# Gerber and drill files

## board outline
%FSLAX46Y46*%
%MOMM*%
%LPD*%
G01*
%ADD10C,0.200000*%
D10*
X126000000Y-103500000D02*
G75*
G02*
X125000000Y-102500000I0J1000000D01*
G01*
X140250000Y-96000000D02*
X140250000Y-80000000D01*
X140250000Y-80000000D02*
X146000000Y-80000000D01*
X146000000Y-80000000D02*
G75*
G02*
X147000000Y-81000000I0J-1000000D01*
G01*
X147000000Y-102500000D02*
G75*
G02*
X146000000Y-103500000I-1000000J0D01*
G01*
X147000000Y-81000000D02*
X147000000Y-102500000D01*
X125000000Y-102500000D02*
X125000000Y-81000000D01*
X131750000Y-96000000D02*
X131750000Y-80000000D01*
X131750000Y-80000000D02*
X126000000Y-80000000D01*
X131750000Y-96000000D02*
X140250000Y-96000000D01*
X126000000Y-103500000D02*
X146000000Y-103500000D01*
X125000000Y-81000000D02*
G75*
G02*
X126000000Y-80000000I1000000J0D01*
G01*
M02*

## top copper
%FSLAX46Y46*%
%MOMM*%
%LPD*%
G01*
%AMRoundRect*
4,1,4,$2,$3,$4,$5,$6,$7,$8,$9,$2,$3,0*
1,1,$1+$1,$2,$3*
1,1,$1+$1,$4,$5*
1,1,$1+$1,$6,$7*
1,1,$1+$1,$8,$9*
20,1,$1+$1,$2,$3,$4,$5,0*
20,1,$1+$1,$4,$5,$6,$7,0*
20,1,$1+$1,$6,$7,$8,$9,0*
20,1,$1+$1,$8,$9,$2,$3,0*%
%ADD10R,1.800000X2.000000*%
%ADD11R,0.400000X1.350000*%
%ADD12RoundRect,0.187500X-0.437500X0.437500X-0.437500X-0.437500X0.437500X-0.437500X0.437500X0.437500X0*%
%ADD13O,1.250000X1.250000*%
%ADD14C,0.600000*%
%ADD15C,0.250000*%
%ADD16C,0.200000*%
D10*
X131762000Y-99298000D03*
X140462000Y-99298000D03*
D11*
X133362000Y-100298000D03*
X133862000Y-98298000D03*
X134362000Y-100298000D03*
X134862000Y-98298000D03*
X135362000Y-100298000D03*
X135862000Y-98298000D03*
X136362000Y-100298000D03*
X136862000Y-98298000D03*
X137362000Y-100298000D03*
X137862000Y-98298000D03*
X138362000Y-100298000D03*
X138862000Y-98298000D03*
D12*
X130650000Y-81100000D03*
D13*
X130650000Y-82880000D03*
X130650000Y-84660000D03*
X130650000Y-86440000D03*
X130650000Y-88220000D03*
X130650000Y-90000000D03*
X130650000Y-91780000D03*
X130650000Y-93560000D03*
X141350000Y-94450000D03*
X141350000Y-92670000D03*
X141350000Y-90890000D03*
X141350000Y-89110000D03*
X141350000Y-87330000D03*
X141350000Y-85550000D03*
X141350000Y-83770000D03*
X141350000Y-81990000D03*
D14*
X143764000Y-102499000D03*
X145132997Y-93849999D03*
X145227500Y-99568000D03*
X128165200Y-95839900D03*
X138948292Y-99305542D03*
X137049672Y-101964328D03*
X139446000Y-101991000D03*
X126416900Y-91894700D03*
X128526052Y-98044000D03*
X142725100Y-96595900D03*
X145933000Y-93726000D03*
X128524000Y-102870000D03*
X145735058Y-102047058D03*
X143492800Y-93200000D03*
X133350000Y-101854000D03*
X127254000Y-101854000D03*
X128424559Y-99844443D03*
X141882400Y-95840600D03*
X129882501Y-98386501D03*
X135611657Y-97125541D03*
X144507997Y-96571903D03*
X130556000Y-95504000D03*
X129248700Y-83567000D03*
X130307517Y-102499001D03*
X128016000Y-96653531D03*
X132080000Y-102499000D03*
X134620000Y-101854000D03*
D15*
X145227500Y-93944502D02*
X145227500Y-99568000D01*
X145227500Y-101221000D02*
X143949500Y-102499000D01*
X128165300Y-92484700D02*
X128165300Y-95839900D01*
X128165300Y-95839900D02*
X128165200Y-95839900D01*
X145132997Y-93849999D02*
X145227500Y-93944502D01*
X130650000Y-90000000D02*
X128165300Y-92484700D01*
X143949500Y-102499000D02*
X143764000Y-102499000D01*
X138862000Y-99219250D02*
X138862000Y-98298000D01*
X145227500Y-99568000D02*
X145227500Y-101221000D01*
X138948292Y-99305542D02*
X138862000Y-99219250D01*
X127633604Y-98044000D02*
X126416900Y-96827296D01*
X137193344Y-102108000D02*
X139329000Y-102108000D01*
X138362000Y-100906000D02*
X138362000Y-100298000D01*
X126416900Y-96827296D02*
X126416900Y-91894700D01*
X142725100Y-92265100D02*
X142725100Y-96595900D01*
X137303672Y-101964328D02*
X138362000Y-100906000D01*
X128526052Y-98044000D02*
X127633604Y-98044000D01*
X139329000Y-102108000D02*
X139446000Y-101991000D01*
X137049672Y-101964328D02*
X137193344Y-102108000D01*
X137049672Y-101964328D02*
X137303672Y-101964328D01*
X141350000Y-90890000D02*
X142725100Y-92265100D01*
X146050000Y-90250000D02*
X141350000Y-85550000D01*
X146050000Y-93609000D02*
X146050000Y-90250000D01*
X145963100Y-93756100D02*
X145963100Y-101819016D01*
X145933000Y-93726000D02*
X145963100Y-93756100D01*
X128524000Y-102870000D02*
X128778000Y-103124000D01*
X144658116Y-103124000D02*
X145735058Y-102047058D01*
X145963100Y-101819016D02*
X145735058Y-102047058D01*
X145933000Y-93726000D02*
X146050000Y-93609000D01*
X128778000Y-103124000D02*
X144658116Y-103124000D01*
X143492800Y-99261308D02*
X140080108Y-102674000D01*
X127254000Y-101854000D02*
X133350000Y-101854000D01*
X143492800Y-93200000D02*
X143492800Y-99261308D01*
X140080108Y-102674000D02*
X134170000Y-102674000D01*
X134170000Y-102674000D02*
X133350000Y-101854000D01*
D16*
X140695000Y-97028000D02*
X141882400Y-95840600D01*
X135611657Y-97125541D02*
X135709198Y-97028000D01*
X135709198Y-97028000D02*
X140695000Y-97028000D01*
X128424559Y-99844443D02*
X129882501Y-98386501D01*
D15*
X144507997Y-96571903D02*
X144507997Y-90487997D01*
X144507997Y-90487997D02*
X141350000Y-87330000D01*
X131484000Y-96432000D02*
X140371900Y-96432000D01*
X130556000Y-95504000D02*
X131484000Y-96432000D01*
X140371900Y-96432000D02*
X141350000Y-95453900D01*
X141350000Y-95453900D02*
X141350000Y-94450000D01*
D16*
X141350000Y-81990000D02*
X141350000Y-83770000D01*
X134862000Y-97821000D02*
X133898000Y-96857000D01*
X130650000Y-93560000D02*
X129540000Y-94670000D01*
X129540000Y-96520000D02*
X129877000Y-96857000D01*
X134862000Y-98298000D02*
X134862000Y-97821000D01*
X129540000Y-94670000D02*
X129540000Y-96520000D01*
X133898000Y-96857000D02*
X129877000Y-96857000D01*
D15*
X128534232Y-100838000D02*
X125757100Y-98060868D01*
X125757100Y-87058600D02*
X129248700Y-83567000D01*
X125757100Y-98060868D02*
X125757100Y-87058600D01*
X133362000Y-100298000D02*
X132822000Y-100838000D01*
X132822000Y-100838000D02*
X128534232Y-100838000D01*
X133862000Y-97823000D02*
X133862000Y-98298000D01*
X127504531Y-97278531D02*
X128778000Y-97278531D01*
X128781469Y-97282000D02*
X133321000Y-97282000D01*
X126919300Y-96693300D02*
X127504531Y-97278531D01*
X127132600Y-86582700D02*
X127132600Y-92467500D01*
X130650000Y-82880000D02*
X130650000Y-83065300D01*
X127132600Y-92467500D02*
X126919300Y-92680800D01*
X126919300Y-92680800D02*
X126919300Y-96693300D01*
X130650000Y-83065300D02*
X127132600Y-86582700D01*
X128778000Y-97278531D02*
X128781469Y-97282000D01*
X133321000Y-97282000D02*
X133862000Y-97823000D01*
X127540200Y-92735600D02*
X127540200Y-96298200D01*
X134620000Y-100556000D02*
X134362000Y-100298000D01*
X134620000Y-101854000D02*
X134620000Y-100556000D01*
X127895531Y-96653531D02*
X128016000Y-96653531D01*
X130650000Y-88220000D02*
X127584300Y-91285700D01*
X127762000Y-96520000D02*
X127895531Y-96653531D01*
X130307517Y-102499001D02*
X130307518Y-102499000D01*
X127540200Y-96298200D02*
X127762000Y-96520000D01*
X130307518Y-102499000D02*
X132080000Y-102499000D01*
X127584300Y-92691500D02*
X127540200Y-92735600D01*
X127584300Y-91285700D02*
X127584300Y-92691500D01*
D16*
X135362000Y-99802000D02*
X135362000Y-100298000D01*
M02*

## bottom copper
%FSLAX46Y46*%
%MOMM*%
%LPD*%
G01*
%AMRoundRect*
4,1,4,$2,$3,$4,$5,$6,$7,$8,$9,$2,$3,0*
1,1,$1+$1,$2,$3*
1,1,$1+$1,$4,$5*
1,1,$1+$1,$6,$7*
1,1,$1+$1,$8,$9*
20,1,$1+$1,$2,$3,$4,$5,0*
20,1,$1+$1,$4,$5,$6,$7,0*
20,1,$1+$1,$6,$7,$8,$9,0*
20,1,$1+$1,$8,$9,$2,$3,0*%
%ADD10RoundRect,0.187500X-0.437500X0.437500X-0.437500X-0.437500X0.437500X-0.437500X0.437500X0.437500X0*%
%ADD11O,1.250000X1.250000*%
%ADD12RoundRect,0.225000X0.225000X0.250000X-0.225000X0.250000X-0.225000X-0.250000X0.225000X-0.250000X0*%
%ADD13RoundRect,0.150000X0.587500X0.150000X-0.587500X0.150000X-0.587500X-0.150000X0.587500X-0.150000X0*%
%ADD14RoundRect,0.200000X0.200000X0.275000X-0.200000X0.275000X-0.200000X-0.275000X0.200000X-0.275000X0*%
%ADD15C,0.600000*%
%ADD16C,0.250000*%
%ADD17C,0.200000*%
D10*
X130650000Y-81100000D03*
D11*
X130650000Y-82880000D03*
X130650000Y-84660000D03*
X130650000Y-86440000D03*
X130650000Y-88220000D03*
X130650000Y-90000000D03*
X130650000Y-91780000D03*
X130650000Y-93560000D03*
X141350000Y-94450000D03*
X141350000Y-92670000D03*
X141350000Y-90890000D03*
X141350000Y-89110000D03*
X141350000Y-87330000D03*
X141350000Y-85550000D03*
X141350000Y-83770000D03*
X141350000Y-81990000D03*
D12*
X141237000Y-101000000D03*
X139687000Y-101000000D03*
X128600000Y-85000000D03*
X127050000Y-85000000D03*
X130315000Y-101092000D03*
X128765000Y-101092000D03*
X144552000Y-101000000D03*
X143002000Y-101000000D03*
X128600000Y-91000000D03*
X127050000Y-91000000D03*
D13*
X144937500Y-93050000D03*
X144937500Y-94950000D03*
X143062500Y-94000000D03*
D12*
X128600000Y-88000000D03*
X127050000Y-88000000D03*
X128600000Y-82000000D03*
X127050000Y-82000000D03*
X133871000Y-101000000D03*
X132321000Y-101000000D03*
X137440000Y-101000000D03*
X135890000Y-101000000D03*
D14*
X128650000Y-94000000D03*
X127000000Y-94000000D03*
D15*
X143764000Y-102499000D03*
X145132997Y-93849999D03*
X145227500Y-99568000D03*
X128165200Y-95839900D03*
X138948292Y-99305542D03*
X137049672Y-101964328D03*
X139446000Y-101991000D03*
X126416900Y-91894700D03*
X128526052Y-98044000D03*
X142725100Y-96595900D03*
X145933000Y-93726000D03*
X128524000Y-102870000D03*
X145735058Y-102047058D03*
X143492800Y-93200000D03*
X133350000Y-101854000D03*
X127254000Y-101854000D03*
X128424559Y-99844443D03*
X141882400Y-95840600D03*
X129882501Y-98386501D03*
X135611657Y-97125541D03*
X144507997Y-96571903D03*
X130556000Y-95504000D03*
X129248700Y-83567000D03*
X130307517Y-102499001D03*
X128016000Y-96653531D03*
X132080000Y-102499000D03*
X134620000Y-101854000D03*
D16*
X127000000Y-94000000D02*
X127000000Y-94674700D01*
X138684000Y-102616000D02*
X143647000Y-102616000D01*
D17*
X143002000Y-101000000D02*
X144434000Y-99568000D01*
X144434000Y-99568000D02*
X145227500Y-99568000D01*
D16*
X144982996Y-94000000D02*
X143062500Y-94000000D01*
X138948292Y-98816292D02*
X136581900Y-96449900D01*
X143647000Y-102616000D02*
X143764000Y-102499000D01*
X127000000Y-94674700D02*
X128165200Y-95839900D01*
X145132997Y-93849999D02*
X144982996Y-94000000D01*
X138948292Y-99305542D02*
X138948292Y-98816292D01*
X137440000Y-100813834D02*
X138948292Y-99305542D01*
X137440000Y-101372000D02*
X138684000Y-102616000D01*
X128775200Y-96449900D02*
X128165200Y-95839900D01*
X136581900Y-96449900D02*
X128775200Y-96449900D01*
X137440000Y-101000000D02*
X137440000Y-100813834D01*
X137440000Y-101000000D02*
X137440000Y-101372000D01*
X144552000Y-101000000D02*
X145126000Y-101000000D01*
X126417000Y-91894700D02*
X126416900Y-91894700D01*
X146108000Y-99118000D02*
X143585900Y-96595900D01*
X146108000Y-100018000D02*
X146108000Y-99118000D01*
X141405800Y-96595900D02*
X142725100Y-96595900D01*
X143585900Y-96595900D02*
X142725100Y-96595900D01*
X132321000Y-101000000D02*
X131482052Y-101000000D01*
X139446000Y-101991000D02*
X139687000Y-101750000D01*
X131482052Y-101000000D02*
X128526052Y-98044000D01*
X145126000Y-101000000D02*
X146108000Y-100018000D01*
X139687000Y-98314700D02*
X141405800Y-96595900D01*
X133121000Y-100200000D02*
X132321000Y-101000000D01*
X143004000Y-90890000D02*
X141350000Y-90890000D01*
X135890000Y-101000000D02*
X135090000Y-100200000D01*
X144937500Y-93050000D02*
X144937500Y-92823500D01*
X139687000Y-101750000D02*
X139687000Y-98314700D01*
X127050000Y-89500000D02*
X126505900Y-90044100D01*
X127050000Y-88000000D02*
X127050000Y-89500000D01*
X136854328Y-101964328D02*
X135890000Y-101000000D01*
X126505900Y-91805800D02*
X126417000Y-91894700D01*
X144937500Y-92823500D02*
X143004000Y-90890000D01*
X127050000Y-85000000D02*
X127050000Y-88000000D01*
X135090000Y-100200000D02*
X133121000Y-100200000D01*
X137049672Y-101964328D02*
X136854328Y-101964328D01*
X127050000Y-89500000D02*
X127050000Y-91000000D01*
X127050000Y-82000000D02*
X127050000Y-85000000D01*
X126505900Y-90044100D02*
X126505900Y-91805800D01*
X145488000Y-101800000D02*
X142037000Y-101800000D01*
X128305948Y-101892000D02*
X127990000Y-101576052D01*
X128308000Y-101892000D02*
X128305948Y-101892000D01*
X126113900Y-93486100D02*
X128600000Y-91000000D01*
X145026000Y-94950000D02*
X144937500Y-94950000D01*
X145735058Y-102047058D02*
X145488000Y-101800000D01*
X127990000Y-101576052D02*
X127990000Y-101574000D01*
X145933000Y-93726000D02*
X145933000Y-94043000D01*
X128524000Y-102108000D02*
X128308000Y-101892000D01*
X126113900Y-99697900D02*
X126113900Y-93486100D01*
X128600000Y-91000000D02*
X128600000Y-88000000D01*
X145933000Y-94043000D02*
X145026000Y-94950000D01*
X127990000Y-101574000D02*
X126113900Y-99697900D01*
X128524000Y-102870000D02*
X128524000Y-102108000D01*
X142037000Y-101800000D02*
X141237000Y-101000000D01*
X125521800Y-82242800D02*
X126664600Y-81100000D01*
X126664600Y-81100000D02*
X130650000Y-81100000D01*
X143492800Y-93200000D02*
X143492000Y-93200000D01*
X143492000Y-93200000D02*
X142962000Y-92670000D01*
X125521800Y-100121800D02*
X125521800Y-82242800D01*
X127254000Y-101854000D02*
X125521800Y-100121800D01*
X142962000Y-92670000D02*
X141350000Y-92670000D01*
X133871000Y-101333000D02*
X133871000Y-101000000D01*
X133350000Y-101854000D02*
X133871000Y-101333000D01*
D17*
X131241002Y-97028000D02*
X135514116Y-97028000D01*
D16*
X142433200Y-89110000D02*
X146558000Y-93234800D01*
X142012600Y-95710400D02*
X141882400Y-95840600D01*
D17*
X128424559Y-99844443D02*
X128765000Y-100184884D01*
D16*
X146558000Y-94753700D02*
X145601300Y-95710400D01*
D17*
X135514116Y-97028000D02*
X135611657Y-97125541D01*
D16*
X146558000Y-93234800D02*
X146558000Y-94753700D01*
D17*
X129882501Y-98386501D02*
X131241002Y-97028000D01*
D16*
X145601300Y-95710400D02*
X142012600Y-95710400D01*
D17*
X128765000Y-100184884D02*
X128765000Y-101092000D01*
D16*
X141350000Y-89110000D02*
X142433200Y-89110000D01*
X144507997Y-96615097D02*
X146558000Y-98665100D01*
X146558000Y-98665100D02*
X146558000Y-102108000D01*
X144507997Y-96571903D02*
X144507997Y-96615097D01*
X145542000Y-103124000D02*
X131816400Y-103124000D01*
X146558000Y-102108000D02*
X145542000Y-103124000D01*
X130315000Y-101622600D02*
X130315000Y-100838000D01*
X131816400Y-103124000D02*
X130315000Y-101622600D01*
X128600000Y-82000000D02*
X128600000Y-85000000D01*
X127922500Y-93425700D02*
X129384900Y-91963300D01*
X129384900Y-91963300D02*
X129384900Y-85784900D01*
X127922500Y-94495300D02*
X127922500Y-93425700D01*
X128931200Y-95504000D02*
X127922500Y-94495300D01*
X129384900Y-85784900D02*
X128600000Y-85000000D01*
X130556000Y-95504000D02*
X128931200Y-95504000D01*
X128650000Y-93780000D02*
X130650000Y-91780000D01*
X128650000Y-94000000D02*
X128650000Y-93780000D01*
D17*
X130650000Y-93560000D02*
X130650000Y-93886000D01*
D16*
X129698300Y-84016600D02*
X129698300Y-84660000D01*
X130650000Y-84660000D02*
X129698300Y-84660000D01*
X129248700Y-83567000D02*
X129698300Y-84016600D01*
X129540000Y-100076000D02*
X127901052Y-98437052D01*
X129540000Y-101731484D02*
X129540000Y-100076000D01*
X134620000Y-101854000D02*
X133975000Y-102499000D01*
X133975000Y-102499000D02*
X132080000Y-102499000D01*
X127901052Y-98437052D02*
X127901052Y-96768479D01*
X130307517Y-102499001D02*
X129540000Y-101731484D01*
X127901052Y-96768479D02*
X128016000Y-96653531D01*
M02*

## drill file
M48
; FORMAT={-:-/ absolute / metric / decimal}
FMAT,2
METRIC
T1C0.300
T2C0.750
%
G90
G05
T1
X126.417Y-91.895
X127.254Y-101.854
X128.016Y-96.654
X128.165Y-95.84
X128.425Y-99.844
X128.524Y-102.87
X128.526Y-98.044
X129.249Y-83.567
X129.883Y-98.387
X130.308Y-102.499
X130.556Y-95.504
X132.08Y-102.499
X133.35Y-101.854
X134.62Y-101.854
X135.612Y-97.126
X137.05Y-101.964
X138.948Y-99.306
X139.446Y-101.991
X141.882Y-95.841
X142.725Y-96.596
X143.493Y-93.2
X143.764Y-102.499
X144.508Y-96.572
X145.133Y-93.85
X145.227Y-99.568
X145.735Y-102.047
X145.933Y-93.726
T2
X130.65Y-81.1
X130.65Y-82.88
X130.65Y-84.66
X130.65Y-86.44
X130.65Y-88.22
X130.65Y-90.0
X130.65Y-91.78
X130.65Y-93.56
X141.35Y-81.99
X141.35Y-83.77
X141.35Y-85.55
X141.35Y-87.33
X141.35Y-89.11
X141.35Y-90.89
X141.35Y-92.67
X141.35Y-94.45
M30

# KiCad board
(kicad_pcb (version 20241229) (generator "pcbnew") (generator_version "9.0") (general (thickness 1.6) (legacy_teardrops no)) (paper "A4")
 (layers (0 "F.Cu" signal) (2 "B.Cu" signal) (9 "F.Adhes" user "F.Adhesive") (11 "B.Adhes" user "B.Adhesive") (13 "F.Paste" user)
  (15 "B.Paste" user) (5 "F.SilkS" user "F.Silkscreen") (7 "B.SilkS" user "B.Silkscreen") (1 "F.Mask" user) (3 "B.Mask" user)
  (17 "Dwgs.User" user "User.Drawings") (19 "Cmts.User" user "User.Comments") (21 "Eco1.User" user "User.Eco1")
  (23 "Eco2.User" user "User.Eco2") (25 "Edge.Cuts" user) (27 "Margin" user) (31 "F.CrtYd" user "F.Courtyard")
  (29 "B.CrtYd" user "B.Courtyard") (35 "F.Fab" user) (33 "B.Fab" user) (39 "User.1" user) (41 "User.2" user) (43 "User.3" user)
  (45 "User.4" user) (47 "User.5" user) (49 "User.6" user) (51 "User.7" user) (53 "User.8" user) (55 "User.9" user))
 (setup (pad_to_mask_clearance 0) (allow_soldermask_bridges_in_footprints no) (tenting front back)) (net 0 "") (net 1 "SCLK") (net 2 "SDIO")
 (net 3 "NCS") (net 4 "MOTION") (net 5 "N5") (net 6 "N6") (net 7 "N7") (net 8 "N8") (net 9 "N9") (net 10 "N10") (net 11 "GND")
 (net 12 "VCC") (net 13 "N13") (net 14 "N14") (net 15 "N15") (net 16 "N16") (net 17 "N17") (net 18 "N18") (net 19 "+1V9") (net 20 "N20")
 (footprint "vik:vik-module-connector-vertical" (layer "F.Cu") (at 136.112 99.298)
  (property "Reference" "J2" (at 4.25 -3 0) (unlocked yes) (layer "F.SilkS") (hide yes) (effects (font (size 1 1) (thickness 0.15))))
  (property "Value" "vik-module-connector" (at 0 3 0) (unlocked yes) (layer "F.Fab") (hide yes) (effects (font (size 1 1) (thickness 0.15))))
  (pad "" smd rect (at -4.35 0) (size 1.8 2) (layers "F.Cu" "F.Mask" "F.Paste") (thermal_bridge_angle 45))
  (pad "" smd rect (at 4.35 0) (size 1.8 2) (layers "F.Cu" "F.Mask" "F.Paste") (thermal_bridge_angle 45))
  (pad "1" smd rect (at -2.75 1) (size 0.4 1.35) (layers "F.Cu" "F.Mask" "F.Paste") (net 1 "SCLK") (thermal_bridge_angle 45))
  (pad "2" smd rect (at -2.25 -1) (size 0.4 1.35) (layers "F.Cu" "F.Mask" "F.Paste") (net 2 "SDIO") (thermal_bridge_angle 45))
  (pad "3" smd rect (at -1.75 1) (size 0.4 1.35) (layers "F.Cu" "F.Mask" "F.Paste") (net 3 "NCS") (thermal_bridge_angle 45))
  (pad "4" smd rect (at -1.25 -1) (size 0.4 1.35) (layers "F.Cu" "F.Mask" "F.Paste") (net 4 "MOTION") (thermal_bridge_angle 45))
  (pad "5" smd rect (at -0.75 1) (size 0.4 1.35) (layers "F.Cu" "F.Mask" "F.Paste") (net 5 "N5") (thermal_bridge_angle 45))
  (pad "6" smd rect (at -0.25 -1) (size 0.4 1.35) (layers "F.Cu" "F.Mask" "F.Paste") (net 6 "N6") (thermal_bridge_angle 45))
  (pad "7" smd rect (at 0.25 1) (size 0.4 1.35) (layers "F.Cu" "F.Mask" "F.Paste") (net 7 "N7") (thermal_bridge_angle 45))
  (pad "8" smd rect (at 0.75 -1) (size 0.4 1.35) (layers "F.Cu" "F.Mask" "F.Paste") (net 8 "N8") (thermal_bridge_angle 45))
  (pad "9" smd rect (at 1.25 1) (size 0.4 1.35) (layers "F.Cu" "F.Mask" "F.Paste") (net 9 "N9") (thermal_bridge_angle 45))
  (pad "10" smd rect (at 1.75 -1) (size 0.4 1.35) (layers "F.Cu" "F.Mask" "F.Paste") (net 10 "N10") (thermal_bridge_angle 45))
  (pad "11" smd rect (at 2.25 1) (size 0.4 1.35) (layers "F.Cu" "F.Mask" "F.Paste") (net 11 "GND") (thermal_bridge_angle 45))
  (pad "12" smd rect (at 2.75 -1) (size 0.4 1.35) (layers "F.Cu" "F.Mask" "F.Paste") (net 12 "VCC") (thermal_bridge_angle 45)))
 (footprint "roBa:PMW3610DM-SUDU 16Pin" (layer "F.Cu") (at 136 87.268 90)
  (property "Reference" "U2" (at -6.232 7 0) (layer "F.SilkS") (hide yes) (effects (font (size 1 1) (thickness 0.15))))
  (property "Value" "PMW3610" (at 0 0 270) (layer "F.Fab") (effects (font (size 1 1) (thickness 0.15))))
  (pad "1" thru_hole roundrect (at 6.168 -5.35 270) (size 1.25 1.25) (drill 0.75) (layers "*.Cu" "*.Mask") (remove_unused_layers no)
   (roundrect_rratio 0.15) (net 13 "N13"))
  (pad "2" thru_hole oval (at 4.388 -5.35 270) (size 1.25 1.25) (drill 0.75) (layers "*.Cu" "*.Mask") (remove_unused_layers no)
   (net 2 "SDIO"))
  (pad "3" thru_hole oval (at 2.608 -5.35 270) (size 1.25 1.25) (drill 0.75) (layers "*.Cu" "*.Mask") (remove_unused_layers no)
   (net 1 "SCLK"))
  (pad "4" thru_hole oval (at 0.828 -5.35 270) (size 1.25 1.25) (drill 0.75) (layers "*.Cu" "*.Mask") (remove_unused_layers no)
   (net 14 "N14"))
  (pad "5" thru_hole oval (at -0.952 -5.35 270) (size 1.25 1.25) (drill 0.75) (layers "*.Cu" "*.Mask") (remove_unused_layers no)
   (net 3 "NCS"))
  (pad "6" thru_hole oval (at -2.732 -5.35 270) (size 1.25 1.25) (drill 0.75) (layers "*.Cu" "*.Mask") (remove_unused_layers no)
   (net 12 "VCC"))
  (pad "7" thru_hole oval (at -4.512 -5.35 270) (size 1.25 1.25) (drill 0.75) (layers "*.Cu" "*.Mask") (remove_unused_layers no)
   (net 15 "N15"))
  (pad "8" thru_hole oval (at -6.292 -5.35 270) (size 1.25 1.25) (drill 0.75) (layers "*.Cu" "*.Mask") (remove_unused_layers no)
   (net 4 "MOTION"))
  (pad "9" thru_hole oval (at -7.182 5.35 270) (size 1.25 1.25) (drill 0.75) (layers "*.Cu" "*.Mask") (remove_unused_layers no)
   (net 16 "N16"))
  (pad "10" thru_hole oval (at -5.402 5.35 270) (size 1.25 1.25) (drill 0.75) (layers "*.Cu" "*.Mask") (remove_unused_layers no)
   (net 13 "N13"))
  (pad "11" thru_hole oval (at -3.622 5.35 270) (size 1.25 1.25) (drill 0.75) (layers "*.Cu" "*.Mask") (remove_unused_layers no)
   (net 11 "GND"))
  (pad "12" thru_hole oval (at -1.842 5.35 270) (size 1.25 1.25) (drill 0.75) (layers "*.Cu" "*.Mask") (remove_unused_layers no)
   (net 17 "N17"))
  (pad "13" thru_hole oval (at -0.062 5.35 270) (size 1.25 1.25) (drill 0.75) (layers "*.Cu" "*.Mask") (remove_unused_layers no)
   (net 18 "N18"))
  (pad "14" thru_hole oval (at 1.718 5.35 270) (size 1.25 1.25) (drill 0.75) (layers "*.Cu" "*.Mask") (remove_unused_layers no)
   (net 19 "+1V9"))
  (pad "15" thru_hole oval (at 3.498 5.35 270) (size 1.25 1.25) (drill 0.75) (layers "*.Cu" "*.Mask") (remove_unused_layers no)
   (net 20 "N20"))
  (pad "16" thru_hole oval (at 5.278 5.35 270) (size 1.25 1.25) (drill 0.75) (layers "*.Cu" "*.Mask") (remove_unused_layers no)
   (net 20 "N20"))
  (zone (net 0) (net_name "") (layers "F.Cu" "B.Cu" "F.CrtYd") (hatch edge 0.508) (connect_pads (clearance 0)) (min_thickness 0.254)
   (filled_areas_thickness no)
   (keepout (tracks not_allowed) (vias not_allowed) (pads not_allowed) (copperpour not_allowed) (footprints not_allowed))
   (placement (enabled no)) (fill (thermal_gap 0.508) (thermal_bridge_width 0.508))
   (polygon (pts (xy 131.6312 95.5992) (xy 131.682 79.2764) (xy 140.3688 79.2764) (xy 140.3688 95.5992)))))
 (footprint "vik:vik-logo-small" (layer "F.Cu") (at 143.5 84.5)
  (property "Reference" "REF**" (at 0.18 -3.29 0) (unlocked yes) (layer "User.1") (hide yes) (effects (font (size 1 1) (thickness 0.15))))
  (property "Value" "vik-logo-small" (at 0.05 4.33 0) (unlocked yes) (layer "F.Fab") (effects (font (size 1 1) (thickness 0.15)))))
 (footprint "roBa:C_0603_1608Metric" (layer "B.Cu") (at 140.462 101 180)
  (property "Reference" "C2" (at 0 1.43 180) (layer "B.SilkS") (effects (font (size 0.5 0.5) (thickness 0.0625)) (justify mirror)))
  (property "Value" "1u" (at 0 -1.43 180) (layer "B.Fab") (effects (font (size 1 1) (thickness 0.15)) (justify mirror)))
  (pad "1" smd roundrect (at -0.775 0 180) (size 0.9 0.95) (layers "B.Cu" "B.Mask" "B.Paste") (roundrect_rratio 0.25) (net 19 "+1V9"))
  (pad "2" smd roundrect (at 0.775 0 180) (size 0.9 0.95) (layers "B.Cu" "B.Mask" "B.Paste") (roundrect_rratio 0.25) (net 11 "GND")))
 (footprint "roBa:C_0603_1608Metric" (layer "B.Cu") (at 127.825 85 180)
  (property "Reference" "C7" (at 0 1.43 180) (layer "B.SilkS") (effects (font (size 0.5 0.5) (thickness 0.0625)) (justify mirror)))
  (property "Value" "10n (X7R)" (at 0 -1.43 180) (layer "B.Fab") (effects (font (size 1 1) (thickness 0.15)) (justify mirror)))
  (pad "1" smd roundrect (at -0.775 0 180) (size 0.9 0.95) (layers "B.Cu" "B.Mask" "B.Paste") (roundrect_rratio 0.25) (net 16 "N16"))
  (pad "2" smd roundrect (at 0.775 0 180) (size 0.9 0.95) (layers "B.Cu" "B.Mask" "B.Paste") (roundrect_rratio 0.25) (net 11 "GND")))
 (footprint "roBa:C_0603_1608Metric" (layer "B.Cu") (at 129.54 101.092 180)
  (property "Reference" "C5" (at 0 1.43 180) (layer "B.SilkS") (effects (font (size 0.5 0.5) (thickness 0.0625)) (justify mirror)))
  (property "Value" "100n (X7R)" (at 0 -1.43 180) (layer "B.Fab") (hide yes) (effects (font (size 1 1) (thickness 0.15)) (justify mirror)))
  (pad "1" smd roundrect (at -0.775 0 180) (size 0.9 0.95) (layers "B.Cu" "B.Mask" "B.Paste") (roundrect_rratio 0.25) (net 18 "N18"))
  (pad "2" smd roundrect (at 0.775 0 180) (size 0.9 0.95) (layers "B.Cu" "B.Mask" "B.Paste") (roundrect_rratio 0.25) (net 17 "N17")))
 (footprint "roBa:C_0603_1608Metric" (layer "B.Cu") (at 143.777 101 180)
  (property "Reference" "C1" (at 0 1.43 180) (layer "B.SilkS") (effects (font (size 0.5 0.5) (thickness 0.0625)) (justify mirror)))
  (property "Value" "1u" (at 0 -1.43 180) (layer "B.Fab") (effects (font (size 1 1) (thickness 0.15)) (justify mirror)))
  (pad "1" smd roundrect (at -0.775 0 180) (size 0.9 0.95) (layers "B.Cu" "B.Mask" "B.Paste") (roundrect_rratio 0.25) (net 11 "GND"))
  (pad "2" smd roundrect (at 0.775 0 180) (size 0.9 0.95) (layers "B.Cu" "B.Mask" "B.Paste") (roundrect_rratio 0.25) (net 12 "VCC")))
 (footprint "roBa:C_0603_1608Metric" (layer "B.Cu") (at 127.825 91 180)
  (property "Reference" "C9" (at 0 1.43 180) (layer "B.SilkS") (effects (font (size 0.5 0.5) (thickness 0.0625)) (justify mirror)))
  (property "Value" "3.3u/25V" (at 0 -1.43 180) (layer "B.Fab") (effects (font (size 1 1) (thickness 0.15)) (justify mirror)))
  (pad "1" smd roundrect (at -0.775 0 180) (size 0.9 0.95) (layers "B.Cu" "B.Mask" "B.Paste") (roundrect_rratio 0.25) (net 19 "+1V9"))
  (pad "2" smd roundrect (at 0.775 0 180) (size 0.9 0.95) (layers "B.Cu" "B.Mask" "B.Paste") (roundrect_rratio 0.25) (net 11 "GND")))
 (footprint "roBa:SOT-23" (layer "B.Cu") (at 144 94 180)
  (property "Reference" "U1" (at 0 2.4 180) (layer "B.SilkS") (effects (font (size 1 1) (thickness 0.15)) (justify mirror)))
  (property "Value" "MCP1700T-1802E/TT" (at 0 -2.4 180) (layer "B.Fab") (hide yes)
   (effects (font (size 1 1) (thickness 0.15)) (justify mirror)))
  (pad "1" smd roundrect (at -0.9375 0.95 180) (size 1.475 0.6) (layers "B.Cu" "B.Mask" "B.Paste") (roundrect_rratio 0.25) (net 11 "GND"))
  (pad "2" smd roundrect (at -0.9375 -0.95 180) (size 1.475 0.6) (layers "B.Cu" "B.Mask" "B.Paste") (roundrect_rratio 0.25) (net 19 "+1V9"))
  (pad "3" smd roundrect (at 0.9375 0 180) (size 1.475 0.6) (layers "B.Cu" "B.Mask" "B.Paste") (roundrect_rratio 0.25) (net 12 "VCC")))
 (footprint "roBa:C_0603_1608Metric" (layer "B.Cu") (at 127.825 88 180)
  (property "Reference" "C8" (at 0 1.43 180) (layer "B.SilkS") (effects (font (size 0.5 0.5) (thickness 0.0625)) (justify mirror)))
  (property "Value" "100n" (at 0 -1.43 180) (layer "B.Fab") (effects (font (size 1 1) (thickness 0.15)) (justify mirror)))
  (pad "1" smd roundrect (at -0.775 0 180) (size 0.9 0.95) (layers "B.Cu" "B.Mask" "B.Paste") (roundrect_rratio 0.25) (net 19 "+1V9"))
  (pad "2" smd roundrect (at 0.775 0 180) (size 0.9 0.95) (layers "B.Cu" "B.Mask" "B.Paste") (roundrect_rratio 0.25) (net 11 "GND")))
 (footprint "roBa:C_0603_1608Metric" (layer "B.Cu") (at 127.825 82 180)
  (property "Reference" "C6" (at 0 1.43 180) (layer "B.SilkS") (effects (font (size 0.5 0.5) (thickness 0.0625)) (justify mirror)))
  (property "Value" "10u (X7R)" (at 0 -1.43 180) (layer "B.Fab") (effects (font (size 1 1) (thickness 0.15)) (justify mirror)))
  (pad "1" smd roundrect (at -0.775 0 180) (size 0.9 0.95) (layers "B.Cu" "B.Mask" "B.Paste") (roundrect_rratio 0.25) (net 16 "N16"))
  (pad "2" smd roundrect (at 0.775 0 180) (size 0.9 0.95) (layers "B.Cu" "B.Mask" "B.Paste") (roundrect_rratio 0.25) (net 11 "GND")))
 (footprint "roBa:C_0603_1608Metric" (layer "B.Cu") (at 133.096 101 180)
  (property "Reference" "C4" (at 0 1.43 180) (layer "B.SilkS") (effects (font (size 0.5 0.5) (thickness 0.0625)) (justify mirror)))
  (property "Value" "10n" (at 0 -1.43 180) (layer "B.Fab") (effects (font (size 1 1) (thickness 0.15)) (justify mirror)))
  (pad "1" smd roundrect (at -0.775 0 180) (size 0.9 0.95) (layers "B.Cu" "B.Mask" "B.Paste") (roundrect_rratio 0.25) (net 13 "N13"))
  (pad "2" smd roundrect (at 0.775 0 180) (size 0.9 0.95) (layers "B.Cu" "B.Mask" "B.Paste") (roundrect_rratio 0.25) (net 11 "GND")))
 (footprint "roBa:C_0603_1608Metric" (layer "B.Cu") (at 136.665 101 180)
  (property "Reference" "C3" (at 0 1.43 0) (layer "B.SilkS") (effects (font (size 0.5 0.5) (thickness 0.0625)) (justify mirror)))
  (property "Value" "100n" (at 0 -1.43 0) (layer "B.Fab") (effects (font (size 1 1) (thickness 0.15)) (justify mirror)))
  (pad "1" smd roundrect (at -0.775 0 180) (size 0.9 0.95) (layers "B.Cu" "B.Mask" "B.Paste") (roundrect_rratio 0.25) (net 12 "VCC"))
  (pad "2" smd roundrect (at 0.775 0 180) (size 0.9 0.95) (layers "B.Cu" "B.Mask" "B.Paste") (roundrect_rratio 0.25) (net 11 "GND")))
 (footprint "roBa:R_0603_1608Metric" (layer "B.Cu") (at 127.825 94 180)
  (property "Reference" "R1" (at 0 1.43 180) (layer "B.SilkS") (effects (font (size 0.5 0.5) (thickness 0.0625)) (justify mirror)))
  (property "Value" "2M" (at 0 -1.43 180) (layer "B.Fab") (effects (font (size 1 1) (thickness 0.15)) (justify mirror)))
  (pad "1" smd roundrect (at -0.825 0 180) (size 0.8 0.95) (layers "B.Cu" "B.Mask" "B.Paste") (roundrect_rratio 0.25) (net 15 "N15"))
  (pad "2" smd roundrect (at 0.825 0 180) (size 0.8 0.95) (layers "B.Cu" "B.Mask" "B.Paste") (roundrect_rratio 0.25) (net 12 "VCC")))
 (gr_arc (start 126 103.5) (mid 125.292893 103.207107) (end 125 102.5) (stroke (width 0.2) (type default)) (layer "Edge.Cuts"))
 (gr_line (start 140.25 96) (end 140.25 80) (stroke (width 0.2) (type default)) (layer "Edge.Cuts"))
 (gr_line (start 140.25 80) (end 146 80) (stroke (width 0.2) (type default)) (layer "Edge.Cuts"))
 (gr_arc (start 146 80) (mid 146.707107 80.292893) (end 147 81) (stroke (width 0.2) (type default)) (layer "Edge.Cuts"))
 (gr_arc (start 147 102.5) (mid 146.707107 103.207107) (end 146 103.5) (stroke (width 0.2) (type default)) (layer "Edge.Cuts"))
 (gr_line (start 147 81) (end 147 102.5) (stroke (width 0.2) (type default)) (layer "Edge.Cuts"))
 (gr_line (start 125 102.5) (end 125 81) (stroke (width 0.2) (type default)) (layer "Edge.Cuts"))
 (gr_line (start 131.75 96) (end 131.75 80) (stroke (width 0.2) (type default)) (layer "Edge.Cuts"))
 (gr_line (start 131.75 80) (end 126 80) (stroke (width 0.2) (type default)) (layer "Edge.Cuts"))
 (gr_line (start 131.75 96) (end 140.25 96) (stroke (width 0.2) (type default)) (layer "Edge.Cuts"))
 (gr_line (start 126 103.5) (end 146 103.5) (stroke (width 0.2) (type default)) (layer "Edge.Cuts"))
 (gr_arc (start 125 81) (mid 125.292893 80.292893) (end 126 80) (stroke (width 0.2) (type default)) (layer "Edge.Cuts"))
 (segment (start 145.2275 93.944502) (end 145.2275 99.568) (width 0.25) (layer "F.Cu") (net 12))
 (segment (start 145.2275 101.221) (end 143.9495 102.499) (width 0.25) (layer "F.Cu") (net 12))
 (segment (start 128.1653 92.4847) (end 128.1653 95.8399) (width 0.25) (layer "F.Cu") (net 12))
 (segment (start 128.1653 95.8399) (end 128.1652 95.8399) (width 0.25) (layer "F.Cu") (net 12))
 (segment (start 145.132997 93.849999) (end 145.2275 93.944502) (width 0.25) (layer "F.Cu") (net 12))
 (segment (start 130.65 90) (end 128.1653 92.4847) (width 0.25) (layer "F.Cu") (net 12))
 (segment (start 143.9495 102.499) (end 143.764 102.499) (width 0.25) (layer "F.Cu") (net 12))
 (segment (start 138.862 99.21925) (end 138.862 98.298) (width 0.25) (layer "F.Cu") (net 12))
 (segment (start 145.2275 99.568) (end 145.2275 101.221) (width 0.25) (layer "F.Cu") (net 12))
 (segment (start 138.948292 99.305542) (end 138.862 99.21925) (width 0.25) (layer "F.Cu") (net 12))
 (via (at 143.764 102.499) (size 0.6) (drill 0.3) (layers "F.Cu" "B.Cu") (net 12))
 (via (at 145.132997 93.849999) (size 0.6) (drill 0.3) (layers "F.Cu" "B.Cu") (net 12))
 (via (at 145.2275 99.568) (size 0.6) (drill 0.3) (layers "F.Cu" "B.Cu") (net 12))
 (via (at 128.1652 95.8399) (size 0.6) (drill 0.3) (layers "F.Cu" "B.Cu") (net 12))
 (via (at 138.948292 99.305542) (size 0.6) (drill 0.3) (layers "F.Cu" "B.Cu") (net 12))
 (segment (start 127 94) (end 127 94.6747) (width 0.25) (layer "B.Cu") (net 12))
 (segment (start 138.684 102.616) (end 143.647 102.616) (width 0.25) (layer "B.Cu") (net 12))
 (segment (start 143.002 101) (end 144.434 99.568) (width 0.2) (layer "B.Cu") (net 12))
 (segment (start 144.434 99.568) (end 145.2275 99.568) (width 0.2) (layer "B.Cu") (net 12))
 (segment (start 144.982996 94) (end 143.0625 94) (width 0.25) (layer "B.Cu") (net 12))
 (segment (start 138.948292 98.816292) (end 136.5819 96.4499) (width 0.25) (layer "B.Cu") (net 12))
 (segment (start 143.647 102.616) (end 143.764 102.499) (width 0.25) (layer "B.Cu") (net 12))
 (segment (start 127 94.6747) (end 128.1652 95.8399) (width 0.25) (layer "B.Cu") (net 12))
 (segment (start 145.132997 93.849999) (end 144.982996 94) (width 0.25) (layer "B.Cu") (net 12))
 (segment (start 138.948292 99.305542) (end 138.948292 98.816292) (width 0.25) (layer "B.Cu") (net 12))
 (segment (start 137.44 100.813834) (end 138.948292 99.305542) (width 0.25) (layer "B.Cu") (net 12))
 (segment (start 137.44 101.372) (end 138.684 102.616) (width 0.25) (layer "B.Cu") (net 12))
 (segment (start 128.7752 96.4499) (end 128.1652 95.8399) (width 0.25) (layer "B.Cu") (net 12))
 (segment (start 136.5819 96.4499) (end 128.7752 96.4499) (width 0.25) (layer "B.Cu") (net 12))
 (segment (start 137.44 101) (end 137.44 100.813834) (width 0.25) (layer "B.Cu") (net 12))
 (segment (start 137.44 101) (end 137.44 101.372) (width 0.25) (layer "B.Cu") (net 12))
 (segment (start 127.633604 98.044) (end 126.4169 96.827296) (width 0.25) (layer "F.Cu") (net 11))
 (segment (start 137.193344 102.108) (end 139.329 102.108) (width 0.25) (layer "F.Cu") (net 11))
 (segment (start 138.362 100.906) (end 138.362 100.298) (width 0.25) (layer "F.Cu") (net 11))
 (segment (start 126.4169 96.827296) (end 126.4169 91.8947) (width 0.25) (layer "F.Cu") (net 11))
 (segment (start 142.7251 92.2651) (end 142.7251 96.5959) (width 0.25) (layer "F.Cu") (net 11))
 (segment (start 137.303672 101.964328) (end 138.362 100.906) (width 0.25) (layer "F.Cu") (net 11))
 (segment (start 128.526052 98.044) (end 127.633604 98.044) (width 0.25) (layer "F.Cu") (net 11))
 (segment (start 139.329 102.108) (end 139.446 101.991) (width 0.25) (layer "F.Cu") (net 11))
 (segment (start 137.049672 101.964328) (end 137.193344 102.108) (width 0.25) (layer "F.Cu") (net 11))
 (segment (start 137.049672 101.964328) (end 137.303672 101.964328) (width 0.25) (layer "F.Cu") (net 11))
 (segment (start 141.35 90.89) (end 142.7251 92.2651) (width 0.25) (layer "F.Cu") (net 11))
 (via (at 137.049672 101.964328) (size 0.6) (drill 0.3) (layers "F.Cu" "B.Cu") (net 11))
 (via (at 139.446 101.991) (size 0.6) (drill 0.3) (layers "F.Cu" "B.Cu") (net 11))
 (via (at 126.4169 91.8947) (size 0.6) (drill 0.3) (layers "F.Cu" "B.Cu") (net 11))
 (via (at 128.526052 98.044) (size 0.6) (drill 0.3) (layers "F.Cu" "B.Cu") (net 11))
 (via (at 142.7251 96.5959) (size 0.6) (drill 0.3) (layers "F.Cu" "B.Cu") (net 11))
 (segment (start 144.552 101) (end 145.126 101) (width 0.25) (layer "B.Cu") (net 11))
 (segment (start 126.417 91.8947) (end 126.4169 91.8947) (width 0.25) (layer "B.Cu") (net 11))
 (segment (start 146.108 99.118) (end 143.5859 96.5959) (width 0.25) (layer "B.Cu") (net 11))
 (segment (start 146.108 100.018) (end 146.108 99.118) (width 0.25) (layer "B.Cu") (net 11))
 (segment (start 141.4058 96.5959) (end 142.7251 96.5959) (width 0.25) (layer "B.Cu") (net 11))
 (segment (start 143.5859 96.5959) (end 142.7251 96.5959) (width 0.25) (layer "B.Cu") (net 11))
 (segment (start 132.321 101) (end 131.482052 101) (width 0.25) (layer "B.Cu") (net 11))
 (segment (start 139.446 101.991) (end 139.687 101.75) (width 0.25) (layer "B.Cu") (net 11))
 (segment (start 131.482052 101) (end 128.526052 98.044) (width 0.25) (layer "B.Cu") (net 11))
 (segment (start 145.126 101) (end 146.108 100.018) (width 0.25) (layer "B.Cu") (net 11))
 (segment (start 139.687 98.3147) (end 141.4058 96.5959) (width 0.25) (layer "B.Cu") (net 11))
 (segment (start 133.121 100.2) (end 132.321 101) (width 0.25) (layer "B.Cu") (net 11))
 (segment (start 143.004 90.89) (end 141.35 90.89) (width 0.25) (layer "B.Cu") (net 11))
 (segment (start 135.89 101) (end 135.09 100.2) (width 0.25) (layer "B.Cu") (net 11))
 (segment (start 144.9375 93.05) (end 144.9375 92.8235) (width 0.25) (layer "B.Cu") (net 11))
 (segment (start 139.687 101.75) (end 139.687 98.3147) (width 0.25) (layer "B.Cu") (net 11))
 (segment (start 127.05 89.5) (end 126.5059 90.0441) (width 0.25) (layer "B.Cu") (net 11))
 (segment (start 127.05 88) (end 127.05 89.5) (width 0.25) (layer "B.Cu") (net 11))
 (segment (start 136.854328 101.964328) (end 135.89 101) (width 0.25) (layer "B.Cu") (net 11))
 (segment (start 126.5059 91.8058) (end 126.417 91.8947) (width 0.25) (layer "B.Cu") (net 11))
 (segment (start 144.9375 92.8235) (end 143.004 90.89) (width 0.25) (layer "B.Cu") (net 11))
 (segment (start 127.05 85) (end 127.05 88) (width 0.25) (layer "B.Cu") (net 11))
 (segment (start 135.09 100.2) (end 133.121 100.2) (width 0.25) (layer "B.Cu") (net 11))
 (segment (start 137.049672 101.964328) (end 136.854328 101.964328) (width 0.25) (layer "B.Cu") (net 11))
 (segment (start 127.05 89.5) (end 127.05 91) (width 0.25) (layer "B.Cu") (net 11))
 (segment (start 127.05 82) (end 127.05 85) (width 0.25) (layer "B.Cu") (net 11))
 (segment (start 126.5059 90.0441) (end 126.5059 91.8058) (width 0.25) (layer "B.Cu") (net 11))
 (segment (start 146.05 90.25) (end 141.35 85.55) (width 0.25) (layer "F.Cu") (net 19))
 (segment (start 146.05 93.609) (end 146.05 90.25) (width 0.25) (layer "F.Cu") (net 19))
 (segment (start 145.9631 93.7561) (end 145.9631 101.819016) (width 0.25) (layer "F.Cu") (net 19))
 (segment (start 145.933 93.726) (end 145.9631 93.7561) (width 0.25) (layer "F.Cu") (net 19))
 (segment (start 128.524 102.87) (end 128.778 103.124) (width 0.25) (layer "F.Cu") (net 19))
 (segment (start 144.658116 103.124) (end 145.735058 102.047058) (width 0.25) (layer "F.Cu") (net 19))
 (segment (start 145.9631 101.819016) (end 145.735058 102.047058) (width 0.25) (layer "F.Cu") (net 19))
 (segment (start 145.933 93.726) (end 146.05 93.609) (width 0.25) (layer "F.Cu") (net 19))
 (segment (start 128.778 103.124) (end 144.658116 103.124) (width 0.25) (layer "F.Cu") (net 19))
 (via (at 145.933 93.726) (size 0.6) (drill 0.3) (layers "F.Cu" "B.Cu") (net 19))
 (via (at 128.524 102.87) (size 0.6) (drill 0.3) (layers "F.Cu" "B.Cu") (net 19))
 (via (at 145.735058 102.047058) (size 0.6) (drill 0.3) (layers "F.Cu" "B.Cu") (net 19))
 (segment (start 145.488 101.8) (end 142.037 101.8) (width 0.25) (layer "B.Cu") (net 19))
 (segment (start 128.305948 101.892) (end 127.99 101.576052) (width 0.25) (layer "B.Cu") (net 19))
 (segment (start 128.308 101.892) (end 128.305948 101.892) (width 0.25) (layer "B.Cu") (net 19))
 (segment (start 126.1139 93.4861) (end 128.6 91) (width 0.25) (layer "B.Cu") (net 19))
 (segment (start 145.026 94.95) (end 144.9375 94.95) (width 0.25) (layer "B.Cu") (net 19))
 (segment (start 145.735058 102.047058) (end 145.488 101.8) (width 0.25) (layer "B.Cu") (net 19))
 (segment (start 127.99 101.576052) (end 127.99 101.574) (width 0.25) (layer "B.Cu") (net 19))
 (segment (start 145.933 93.726) (end 145.933 94.043) (width 0.25) (layer "B.Cu") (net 19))
 (segment (start 128.524 102.108) (end 128.308 101.892) (width 0.25) (layer "B.Cu") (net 19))
 (segment (start 126.1139 99.6979) (end 126.1139 93.4861) (width 0.25) (layer "B.Cu") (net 19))
 (segment (start 128.6 91) (end 128.6 88) (width 0.25) (layer "B.Cu") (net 19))
 (segment (start 145.933 94.043) (end 145.026 94.95) (width 0.25) (layer "B.Cu") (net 19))
 (segment (start 127.99 101.574) (end 126.1139 99.6979) (width 0.25) (layer "B.Cu") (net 19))
 (segment (start 128.524 102.87) (end 128.524 102.108) (width 0.25) (layer "B.Cu") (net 19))
 (segment (start 142.037 101.8) (end 141.237 101) (width 0.25) (layer "B.Cu") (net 19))
 (segment (start 143.4928 99.261308) (end 140.080108 102.674) (width 0.25) (layer "F.Cu") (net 13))
 (segment (start 127.254 101.854) (end 133.35 101.854) (width 0.25) (layer "F.Cu") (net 13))
 (segment (start 143.4928 93.2) (end 143.4928 99.261308) (width 0.25) (layer "F.Cu") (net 13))
 (segment (start 140.080108 102.674) (end 134.17 102.674) (width 0.25) (layer "F.Cu") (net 13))
 (segment (start 134.17 102.674) (end 133.35 101.854) (width 0.25) (layer "F.Cu") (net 13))
 (via (at 143.4928 93.2) (size 0.6) (drill 0.3) (layers "F.Cu" "B.Cu") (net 13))
 (via (at 133.35 101.854) (size 0.6) (drill 0.3) (layers "F.Cu" "B.Cu") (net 13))
 (via (at 127.254 101.854) (size 0.6) (drill 0.3) (layers "F.Cu" "B.Cu") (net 13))
 (segment (start 125.5218 82.2428) (end 126.6646 81.1) (width 0.25) (layer "B.Cu") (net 13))
 (segment (start 126.6646 81.1) (end 130.65 81.1) (width 0.25) (layer "B.Cu") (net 13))
 (segment (start 143.4928 93.2) (end 143.492 93.2) (width 0.25) (layer "B.Cu") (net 13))
 (segment (start 143.492 93.2) (end 142.962 92.67) (width 0.25) (layer "B.Cu") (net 13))
 (segment (start 125.5218 100.1218) (end 125.5218 82.2428) (width 0.25) (layer "B.Cu") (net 13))
 (segment (start 127.254 101.854) (end 125.5218 100.1218) (width 0.25) (layer "B.Cu") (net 13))
 (segment (start 142.962 92.67) (end 141.35 92.67) (width 0.25) (layer "B.Cu") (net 13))
 (segment (start 133.871 101.333) (end 133.871 101) (width 0.25) (layer "B.Cu") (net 13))
 (segment (start 133.35 101.854) (end 133.871 101.333) (width 0.25) (layer "B.Cu") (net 13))
 (segment (start 140.695 97.028) (end 141.8824 95.8406) (width 0.2) (layer "F.Cu") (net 17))
 (segment (start 135.611657 97.125541) (end 135.709198 97.028) (width 0.2) (layer "F.Cu") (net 17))
 (segment (start 135.709198 97.028) (end 140.695 97.028) (width 0.2) (layer "F.Cu") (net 17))
 (segment (start 128.424559 99.844443) (end 129.882501 98.386501) (width 0.2) (layer "F.Cu") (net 17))
 (via (at 128.424559 99.844443) (size 0.6) (drill 0.3) (layers "F.Cu" "B.Cu") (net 17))
 (via (at 141.8824 95.8406) (size 0.6) (drill 0.3) (layers "F.Cu" "B.Cu") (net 17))
 (via (at 129.882501 98.386501) (size 0.6) (drill 0.3) (layers "F.Cu" "B.Cu") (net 17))
 (via (at 135.611657 97.125541) (size 0.6) (drill 0.3) (layers "F.Cu" "B.Cu") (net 17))
 (segment (start 131.241002 97.028) (end 135.514116 97.028) (width 0.2) (layer "B.Cu") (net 17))
 (segment (start 142.4332 89.11) (end 146.558 93.2348) (width 0.25) (layer "B.Cu") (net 17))
 (segment (start 142.0126 95.7104) (end 141.8824 95.8406) (width 0.25) (layer "B.Cu") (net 17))
 (segment (start 128.424559 99.844443) (end 128.765 100.184884) (width 0.2) (layer "B.Cu") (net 17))
 (segment (start 146.558 94.7537) (end 145.6013 95.7104) (width 0.25) (layer "B.Cu") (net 17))
 (segment (start 135.514116 97.028) (end 135.611657 97.125541) (width 0.2) (layer "B.Cu") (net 17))
 (segment (start 146.558 93.2348) (end 146.558 94.7537) (width 0.25) (layer "B.Cu") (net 17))
 (segment (start 129.882501 98.386501) (end 131.241002 97.028) (width 0.2) (layer "B.Cu") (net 17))
 (segment (start 145.6013 95.7104) (end 142.0126 95.7104) (width 0.25) (layer "B.Cu") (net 17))
 (segment (start 128.765 100.184884) (end 128.765 101.092) (width 0.2) (layer "B.Cu") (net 17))
 (segment (start 141.35 89.11) (end 142.4332 89.11) (width 0.25) (layer "B.Cu") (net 17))
 (segment (start 144.507997 96.571903) (end 144.507997 90.487997) (width 0.25) (layer "F.Cu") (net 18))
 (segment (start 144.507997 90.487997) (end 141.35 87.33) (width 0.25) (layer "F.Cu") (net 18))
 (via (at 144.507997 96.571903) (size 0.6) (drill 0.3) (layers "F.Cu" "B.Cu") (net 18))
 (segment (start 144.507997 96.615097) (end 146.558 98.6651) (width 0.25) (layer "B.Cu") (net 18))
 (segment (start 146.558 98.6651) (end 146.558 102.108) (width 0.25) (layer "B.Cu") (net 18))
 (segment (start 144.507997 96.571903) (end 144.507997 96.615097) (width 0.25) (layer "B.Cu") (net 18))
 (segment (start 145.542 103.124) (end 131.8164 103.124) (width 0.25) (layer "B.Cu") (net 18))
 (segment (start 146.558 102.108) (end 145.542 103.124) (width 0.25) (layer "B.Cu") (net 18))
 (segment (start 130.315 101.6226) (end 130.315 100.838) (width 0.25) (layer "B.Cu") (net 18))
 (segment (start 131.8164 103.124) (end 130.315 101.6226) (width 0.25) (layer "B.Cu") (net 18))
 (segment (start 131.484 96.432) (end 140.3719 96.432) (width 0.25) (layer "F.Cu") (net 16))
 (segment (start 130.556 95.504) (end 131.484 96.432) (width 0.25) (layer "F.Cu") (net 16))
 (segment (start 140.3719 96.432) (end 141.35 95.4539) (width 0.25) (layer "F.Cu") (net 16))
 (segment (start 141.35 95.4539) (end 141.35 94.45) (width 0.25) (layer "F.Cu") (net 16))
 (via (at 130.556 95.504) (size 0.6) (drill 0.3) (layers "F.Cu" "B.Cu") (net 16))
 (segment (start 128.6 82) (end 128.6 85) (width 0.25) (layer "B.Cu") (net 16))
 (segment (start 127.9225 93.4257) (end 129.3849 91.9633) (width 0.25) (layer "B.Cu") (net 16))
 (segment (start 129.3849 91.9633) (end 129.3849 85.7849) (width 0.25) (layer "B.Cu") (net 16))
 (segment (start 127.9225 94.4953) (end 127.9225 93.4257) (width 0.25) (layer "B.Cu") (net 16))
 (segment (start 128.9312 95.504) (end 127.9225 94.4953) (width 0.25) (layer "B.Cu") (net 16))
 (segment (start 129.3849 85.7849) (end 128.6 85) (width 0.25) (layer "B.Cu") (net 16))
 (segment (start 130.556 95.504) (end 128.9312 95.504) (width 0.25) (layer "B.Cu") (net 16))
 (segment (start 128.65 93.78) (end 130.65 91.78) (width 0.25) (layer "B.Cu") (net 15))
 (segment (start 128.65 94) (end 128.65 93.78) (width 0.25) (layer "B.Cu") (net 15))
 (segment (start 141.35 81.99) (end 141.35 83.77) (width 0.2) (layer "F.Cu") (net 20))
 (segment (start 134.862 97.821) (end 133.898 96.857) (width 0.2) (layer "F.Cu") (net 4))
 (segment (start 130.65 93.56) (end 129.54 94.67) (width 0.2) (layer "F.Cu") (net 4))
 (segment (start 129.54 96.52) (end 129.877 96.857) (width 0.2) (layer "F.Cu") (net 4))
 (segment (start 134.862 98.298) (end 134.862 97.821) (width 0.2) (layer "F.Cu") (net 4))
 (segment (start 129.54 94.67) (end 129.54 96.52) (width 0.2) (layer "F.Cu") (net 4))
 (segment (start 133.898 96.857) (end 129.877 96.857) (width 0.2) (layer "F.Cu") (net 4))
 (segment (start 130.65 93.56) (end 130.65 93.886) (width 0.2) (layer "B.Cu") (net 4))
 (segment (start 128.534232 100.838) (end 125.7571 98.060868) (width 0.25) (layer "F.Cu") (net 1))
 (segment (start 125.7571 87.0586) (end 129.2487 83.567) (width 0.25) (layer "F.Cu") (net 1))
 (segment (start 125.7571 98.060868) (end 125.7571 87.0586) (width 0.25) (layer "F.Cu") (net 1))
 (segment (start 133.362 100.298) (end 132.822 100.838) (width 0.25) (layer "F.Cu") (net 1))
 (segment (start 132.822 100.838) (end 128.534232 100.838) (width 0.25) (layer "F.Cu") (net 1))
 (via (at 129.2487 83.567) (size 0.6) (drill 0.3) (layers "F.Cu" "B.Cu") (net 1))
 (segment (start 129.6983 84.0166) (end 129.6983 84.66) (width 0.25) (layer "B.Cu") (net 1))
 (segment (start 130.65 84.66) (end 129.6983 84.66) (width 0.25) (layer "B.Cu") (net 1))
 (segment (start 129.2487 83.567) (end 129.6983 84.0166) (width 0.25) (layer "B.Cu") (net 1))
 (segment (start 133.862 97.823) (end 133.862 98.298) (width 0.25) (layer "F.Cu") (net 2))
 (segment (start 127.504531 97.278531) (end 128.778 97.278531) (width 0.25) (layer "F.Cu") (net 2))
 (segment (start 128.781469 97.282) (end 133.321 97.282) (width 0.25) (layer "F.Cu") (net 2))
 (segment (start 126.9193 96.6933) (end 127.504531 97.278531) (width 0.25) (layer "F.Cu") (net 2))
 (segment (start 127.1326 86.5827) (end 127.1326 92.4675) (width 0.25) (layer "F.Cu") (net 2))
 (segment (start 130.65 82.88) (end 130.65 83.0653) (width 0.25) (layer "F.Cu") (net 2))
 (segment (start 127.1326 92.4675) (end 126.9193 92.6808) (width 0.25) (layer "F.Cu") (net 2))
 (segment (start 126.9193 92.6808) (end 126.9193 96.6933) (width 0.25) (layer "F.Cu") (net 2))
 (segment (start 130.65 83.0653) (end 127.1326 86.5827) (width 0.25) (layer "F.Cu") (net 2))
 (segment (start 128.778 97.278531) (end 128.781469 97.282) (width 0.25) (layer "F.Cu") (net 2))
 (segment (start 133.321 97.282) (end 133.862 97.823) (width 0.25) (layer "F.Cu") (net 2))
 (segment (start 127.5402 92.7356) (end 127.5402 96.2982) (width 0.25) (layer "F.Cu") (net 3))
 (segment (start 134.62 100.556) (end 134.362 100.298) (width 0.25) (layer "F.Cu") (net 3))
 (segment (start 134.62 101.854) (end 134.62 100.556) (width 0.25) (layer "F.Cu") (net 3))
 (segment (start 127.895531 96.653531) (end 128.016 96.653531) (width 0.25) (layer "F.Cu") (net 3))
 (segment (start 130.65 88.22) (end 127.5843 91.2857) (width 0.25) (layer "F.Cu") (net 3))
 (segment (start 127.762 96.52) (end 127.895531 96.653531) (width 0.25) (layer "F.Cu") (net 3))
 (segment (start 130.307517 102.499001) (end 130.307518 102.499) (width 0.25) (layer "F.Cu") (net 3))
 (segment (start 127.5402 96.2982) (end 127.762 96.52) (width 0.25) (layer "F.Cu") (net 3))
 (segment (start 130.307518 102.499) (end 132.08 102.499) (width 0.25) (layer "F.Cu") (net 3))
 (segment (start 127.5843 92.6915) (end 127.5402 92.7356) (width 0.25) (layer "F.Cu") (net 3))
 (segment (start 127.5843 91.2857) (end 127.5843 92.6915) (width 0.25) (layer "F.Cu") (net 3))
 (via (at 130.307517 102.499001) (size 0.6) (drill 0.3) (layers "F.Cu" "B.Cu") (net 3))
 (via (at 128.016 96.653531) (size 0.6) (drill 0.3) (layers "F.Cu" "B.Cu") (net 3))
 (via (at 132.08 102.499) (size 0.6) (drill 0.3) (layers "F.Cu" "B.Cu") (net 3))
 (via (at 134.62 101.854) (size 0.6) (drill 0.3) (layers "F.Cu" "B.Cu") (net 3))
 (segment (start 129.54 100.076) (end 127.901052 98.437052) (width 0.25) (layer "B.Cu") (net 3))
 (segment (start 129.54 101.731484) (end 129.54 100.076) (width 0.25) (layer "B.Cu") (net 3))
 (segment (start 134.62 101.854) (end 133.975 102.499) (width 0.25) (layer "B.Cu") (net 3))
 (segment (start 133.975 102.499) (end 132.08 102.499) (width 0.25) (layer "B.Cu") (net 3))
 (segment (start 127.901052 98.437052) (end 127.901052 96.768479) (width 0.25) (layer "B.Cu") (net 3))
 (segment (start 130.307517 102.499001) (end 129.54 101.731484) (width 0.25) (layer "B.Cu") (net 3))
 (segment (start 127.901052 96.768479) (end 128.016 96.653531) (width 0.25) (layer "B.Cu") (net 3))
 (segment (start 135.362 99.802) (end 135.362 100.298) (width 0.2) (layer "F.Cu") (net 5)))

